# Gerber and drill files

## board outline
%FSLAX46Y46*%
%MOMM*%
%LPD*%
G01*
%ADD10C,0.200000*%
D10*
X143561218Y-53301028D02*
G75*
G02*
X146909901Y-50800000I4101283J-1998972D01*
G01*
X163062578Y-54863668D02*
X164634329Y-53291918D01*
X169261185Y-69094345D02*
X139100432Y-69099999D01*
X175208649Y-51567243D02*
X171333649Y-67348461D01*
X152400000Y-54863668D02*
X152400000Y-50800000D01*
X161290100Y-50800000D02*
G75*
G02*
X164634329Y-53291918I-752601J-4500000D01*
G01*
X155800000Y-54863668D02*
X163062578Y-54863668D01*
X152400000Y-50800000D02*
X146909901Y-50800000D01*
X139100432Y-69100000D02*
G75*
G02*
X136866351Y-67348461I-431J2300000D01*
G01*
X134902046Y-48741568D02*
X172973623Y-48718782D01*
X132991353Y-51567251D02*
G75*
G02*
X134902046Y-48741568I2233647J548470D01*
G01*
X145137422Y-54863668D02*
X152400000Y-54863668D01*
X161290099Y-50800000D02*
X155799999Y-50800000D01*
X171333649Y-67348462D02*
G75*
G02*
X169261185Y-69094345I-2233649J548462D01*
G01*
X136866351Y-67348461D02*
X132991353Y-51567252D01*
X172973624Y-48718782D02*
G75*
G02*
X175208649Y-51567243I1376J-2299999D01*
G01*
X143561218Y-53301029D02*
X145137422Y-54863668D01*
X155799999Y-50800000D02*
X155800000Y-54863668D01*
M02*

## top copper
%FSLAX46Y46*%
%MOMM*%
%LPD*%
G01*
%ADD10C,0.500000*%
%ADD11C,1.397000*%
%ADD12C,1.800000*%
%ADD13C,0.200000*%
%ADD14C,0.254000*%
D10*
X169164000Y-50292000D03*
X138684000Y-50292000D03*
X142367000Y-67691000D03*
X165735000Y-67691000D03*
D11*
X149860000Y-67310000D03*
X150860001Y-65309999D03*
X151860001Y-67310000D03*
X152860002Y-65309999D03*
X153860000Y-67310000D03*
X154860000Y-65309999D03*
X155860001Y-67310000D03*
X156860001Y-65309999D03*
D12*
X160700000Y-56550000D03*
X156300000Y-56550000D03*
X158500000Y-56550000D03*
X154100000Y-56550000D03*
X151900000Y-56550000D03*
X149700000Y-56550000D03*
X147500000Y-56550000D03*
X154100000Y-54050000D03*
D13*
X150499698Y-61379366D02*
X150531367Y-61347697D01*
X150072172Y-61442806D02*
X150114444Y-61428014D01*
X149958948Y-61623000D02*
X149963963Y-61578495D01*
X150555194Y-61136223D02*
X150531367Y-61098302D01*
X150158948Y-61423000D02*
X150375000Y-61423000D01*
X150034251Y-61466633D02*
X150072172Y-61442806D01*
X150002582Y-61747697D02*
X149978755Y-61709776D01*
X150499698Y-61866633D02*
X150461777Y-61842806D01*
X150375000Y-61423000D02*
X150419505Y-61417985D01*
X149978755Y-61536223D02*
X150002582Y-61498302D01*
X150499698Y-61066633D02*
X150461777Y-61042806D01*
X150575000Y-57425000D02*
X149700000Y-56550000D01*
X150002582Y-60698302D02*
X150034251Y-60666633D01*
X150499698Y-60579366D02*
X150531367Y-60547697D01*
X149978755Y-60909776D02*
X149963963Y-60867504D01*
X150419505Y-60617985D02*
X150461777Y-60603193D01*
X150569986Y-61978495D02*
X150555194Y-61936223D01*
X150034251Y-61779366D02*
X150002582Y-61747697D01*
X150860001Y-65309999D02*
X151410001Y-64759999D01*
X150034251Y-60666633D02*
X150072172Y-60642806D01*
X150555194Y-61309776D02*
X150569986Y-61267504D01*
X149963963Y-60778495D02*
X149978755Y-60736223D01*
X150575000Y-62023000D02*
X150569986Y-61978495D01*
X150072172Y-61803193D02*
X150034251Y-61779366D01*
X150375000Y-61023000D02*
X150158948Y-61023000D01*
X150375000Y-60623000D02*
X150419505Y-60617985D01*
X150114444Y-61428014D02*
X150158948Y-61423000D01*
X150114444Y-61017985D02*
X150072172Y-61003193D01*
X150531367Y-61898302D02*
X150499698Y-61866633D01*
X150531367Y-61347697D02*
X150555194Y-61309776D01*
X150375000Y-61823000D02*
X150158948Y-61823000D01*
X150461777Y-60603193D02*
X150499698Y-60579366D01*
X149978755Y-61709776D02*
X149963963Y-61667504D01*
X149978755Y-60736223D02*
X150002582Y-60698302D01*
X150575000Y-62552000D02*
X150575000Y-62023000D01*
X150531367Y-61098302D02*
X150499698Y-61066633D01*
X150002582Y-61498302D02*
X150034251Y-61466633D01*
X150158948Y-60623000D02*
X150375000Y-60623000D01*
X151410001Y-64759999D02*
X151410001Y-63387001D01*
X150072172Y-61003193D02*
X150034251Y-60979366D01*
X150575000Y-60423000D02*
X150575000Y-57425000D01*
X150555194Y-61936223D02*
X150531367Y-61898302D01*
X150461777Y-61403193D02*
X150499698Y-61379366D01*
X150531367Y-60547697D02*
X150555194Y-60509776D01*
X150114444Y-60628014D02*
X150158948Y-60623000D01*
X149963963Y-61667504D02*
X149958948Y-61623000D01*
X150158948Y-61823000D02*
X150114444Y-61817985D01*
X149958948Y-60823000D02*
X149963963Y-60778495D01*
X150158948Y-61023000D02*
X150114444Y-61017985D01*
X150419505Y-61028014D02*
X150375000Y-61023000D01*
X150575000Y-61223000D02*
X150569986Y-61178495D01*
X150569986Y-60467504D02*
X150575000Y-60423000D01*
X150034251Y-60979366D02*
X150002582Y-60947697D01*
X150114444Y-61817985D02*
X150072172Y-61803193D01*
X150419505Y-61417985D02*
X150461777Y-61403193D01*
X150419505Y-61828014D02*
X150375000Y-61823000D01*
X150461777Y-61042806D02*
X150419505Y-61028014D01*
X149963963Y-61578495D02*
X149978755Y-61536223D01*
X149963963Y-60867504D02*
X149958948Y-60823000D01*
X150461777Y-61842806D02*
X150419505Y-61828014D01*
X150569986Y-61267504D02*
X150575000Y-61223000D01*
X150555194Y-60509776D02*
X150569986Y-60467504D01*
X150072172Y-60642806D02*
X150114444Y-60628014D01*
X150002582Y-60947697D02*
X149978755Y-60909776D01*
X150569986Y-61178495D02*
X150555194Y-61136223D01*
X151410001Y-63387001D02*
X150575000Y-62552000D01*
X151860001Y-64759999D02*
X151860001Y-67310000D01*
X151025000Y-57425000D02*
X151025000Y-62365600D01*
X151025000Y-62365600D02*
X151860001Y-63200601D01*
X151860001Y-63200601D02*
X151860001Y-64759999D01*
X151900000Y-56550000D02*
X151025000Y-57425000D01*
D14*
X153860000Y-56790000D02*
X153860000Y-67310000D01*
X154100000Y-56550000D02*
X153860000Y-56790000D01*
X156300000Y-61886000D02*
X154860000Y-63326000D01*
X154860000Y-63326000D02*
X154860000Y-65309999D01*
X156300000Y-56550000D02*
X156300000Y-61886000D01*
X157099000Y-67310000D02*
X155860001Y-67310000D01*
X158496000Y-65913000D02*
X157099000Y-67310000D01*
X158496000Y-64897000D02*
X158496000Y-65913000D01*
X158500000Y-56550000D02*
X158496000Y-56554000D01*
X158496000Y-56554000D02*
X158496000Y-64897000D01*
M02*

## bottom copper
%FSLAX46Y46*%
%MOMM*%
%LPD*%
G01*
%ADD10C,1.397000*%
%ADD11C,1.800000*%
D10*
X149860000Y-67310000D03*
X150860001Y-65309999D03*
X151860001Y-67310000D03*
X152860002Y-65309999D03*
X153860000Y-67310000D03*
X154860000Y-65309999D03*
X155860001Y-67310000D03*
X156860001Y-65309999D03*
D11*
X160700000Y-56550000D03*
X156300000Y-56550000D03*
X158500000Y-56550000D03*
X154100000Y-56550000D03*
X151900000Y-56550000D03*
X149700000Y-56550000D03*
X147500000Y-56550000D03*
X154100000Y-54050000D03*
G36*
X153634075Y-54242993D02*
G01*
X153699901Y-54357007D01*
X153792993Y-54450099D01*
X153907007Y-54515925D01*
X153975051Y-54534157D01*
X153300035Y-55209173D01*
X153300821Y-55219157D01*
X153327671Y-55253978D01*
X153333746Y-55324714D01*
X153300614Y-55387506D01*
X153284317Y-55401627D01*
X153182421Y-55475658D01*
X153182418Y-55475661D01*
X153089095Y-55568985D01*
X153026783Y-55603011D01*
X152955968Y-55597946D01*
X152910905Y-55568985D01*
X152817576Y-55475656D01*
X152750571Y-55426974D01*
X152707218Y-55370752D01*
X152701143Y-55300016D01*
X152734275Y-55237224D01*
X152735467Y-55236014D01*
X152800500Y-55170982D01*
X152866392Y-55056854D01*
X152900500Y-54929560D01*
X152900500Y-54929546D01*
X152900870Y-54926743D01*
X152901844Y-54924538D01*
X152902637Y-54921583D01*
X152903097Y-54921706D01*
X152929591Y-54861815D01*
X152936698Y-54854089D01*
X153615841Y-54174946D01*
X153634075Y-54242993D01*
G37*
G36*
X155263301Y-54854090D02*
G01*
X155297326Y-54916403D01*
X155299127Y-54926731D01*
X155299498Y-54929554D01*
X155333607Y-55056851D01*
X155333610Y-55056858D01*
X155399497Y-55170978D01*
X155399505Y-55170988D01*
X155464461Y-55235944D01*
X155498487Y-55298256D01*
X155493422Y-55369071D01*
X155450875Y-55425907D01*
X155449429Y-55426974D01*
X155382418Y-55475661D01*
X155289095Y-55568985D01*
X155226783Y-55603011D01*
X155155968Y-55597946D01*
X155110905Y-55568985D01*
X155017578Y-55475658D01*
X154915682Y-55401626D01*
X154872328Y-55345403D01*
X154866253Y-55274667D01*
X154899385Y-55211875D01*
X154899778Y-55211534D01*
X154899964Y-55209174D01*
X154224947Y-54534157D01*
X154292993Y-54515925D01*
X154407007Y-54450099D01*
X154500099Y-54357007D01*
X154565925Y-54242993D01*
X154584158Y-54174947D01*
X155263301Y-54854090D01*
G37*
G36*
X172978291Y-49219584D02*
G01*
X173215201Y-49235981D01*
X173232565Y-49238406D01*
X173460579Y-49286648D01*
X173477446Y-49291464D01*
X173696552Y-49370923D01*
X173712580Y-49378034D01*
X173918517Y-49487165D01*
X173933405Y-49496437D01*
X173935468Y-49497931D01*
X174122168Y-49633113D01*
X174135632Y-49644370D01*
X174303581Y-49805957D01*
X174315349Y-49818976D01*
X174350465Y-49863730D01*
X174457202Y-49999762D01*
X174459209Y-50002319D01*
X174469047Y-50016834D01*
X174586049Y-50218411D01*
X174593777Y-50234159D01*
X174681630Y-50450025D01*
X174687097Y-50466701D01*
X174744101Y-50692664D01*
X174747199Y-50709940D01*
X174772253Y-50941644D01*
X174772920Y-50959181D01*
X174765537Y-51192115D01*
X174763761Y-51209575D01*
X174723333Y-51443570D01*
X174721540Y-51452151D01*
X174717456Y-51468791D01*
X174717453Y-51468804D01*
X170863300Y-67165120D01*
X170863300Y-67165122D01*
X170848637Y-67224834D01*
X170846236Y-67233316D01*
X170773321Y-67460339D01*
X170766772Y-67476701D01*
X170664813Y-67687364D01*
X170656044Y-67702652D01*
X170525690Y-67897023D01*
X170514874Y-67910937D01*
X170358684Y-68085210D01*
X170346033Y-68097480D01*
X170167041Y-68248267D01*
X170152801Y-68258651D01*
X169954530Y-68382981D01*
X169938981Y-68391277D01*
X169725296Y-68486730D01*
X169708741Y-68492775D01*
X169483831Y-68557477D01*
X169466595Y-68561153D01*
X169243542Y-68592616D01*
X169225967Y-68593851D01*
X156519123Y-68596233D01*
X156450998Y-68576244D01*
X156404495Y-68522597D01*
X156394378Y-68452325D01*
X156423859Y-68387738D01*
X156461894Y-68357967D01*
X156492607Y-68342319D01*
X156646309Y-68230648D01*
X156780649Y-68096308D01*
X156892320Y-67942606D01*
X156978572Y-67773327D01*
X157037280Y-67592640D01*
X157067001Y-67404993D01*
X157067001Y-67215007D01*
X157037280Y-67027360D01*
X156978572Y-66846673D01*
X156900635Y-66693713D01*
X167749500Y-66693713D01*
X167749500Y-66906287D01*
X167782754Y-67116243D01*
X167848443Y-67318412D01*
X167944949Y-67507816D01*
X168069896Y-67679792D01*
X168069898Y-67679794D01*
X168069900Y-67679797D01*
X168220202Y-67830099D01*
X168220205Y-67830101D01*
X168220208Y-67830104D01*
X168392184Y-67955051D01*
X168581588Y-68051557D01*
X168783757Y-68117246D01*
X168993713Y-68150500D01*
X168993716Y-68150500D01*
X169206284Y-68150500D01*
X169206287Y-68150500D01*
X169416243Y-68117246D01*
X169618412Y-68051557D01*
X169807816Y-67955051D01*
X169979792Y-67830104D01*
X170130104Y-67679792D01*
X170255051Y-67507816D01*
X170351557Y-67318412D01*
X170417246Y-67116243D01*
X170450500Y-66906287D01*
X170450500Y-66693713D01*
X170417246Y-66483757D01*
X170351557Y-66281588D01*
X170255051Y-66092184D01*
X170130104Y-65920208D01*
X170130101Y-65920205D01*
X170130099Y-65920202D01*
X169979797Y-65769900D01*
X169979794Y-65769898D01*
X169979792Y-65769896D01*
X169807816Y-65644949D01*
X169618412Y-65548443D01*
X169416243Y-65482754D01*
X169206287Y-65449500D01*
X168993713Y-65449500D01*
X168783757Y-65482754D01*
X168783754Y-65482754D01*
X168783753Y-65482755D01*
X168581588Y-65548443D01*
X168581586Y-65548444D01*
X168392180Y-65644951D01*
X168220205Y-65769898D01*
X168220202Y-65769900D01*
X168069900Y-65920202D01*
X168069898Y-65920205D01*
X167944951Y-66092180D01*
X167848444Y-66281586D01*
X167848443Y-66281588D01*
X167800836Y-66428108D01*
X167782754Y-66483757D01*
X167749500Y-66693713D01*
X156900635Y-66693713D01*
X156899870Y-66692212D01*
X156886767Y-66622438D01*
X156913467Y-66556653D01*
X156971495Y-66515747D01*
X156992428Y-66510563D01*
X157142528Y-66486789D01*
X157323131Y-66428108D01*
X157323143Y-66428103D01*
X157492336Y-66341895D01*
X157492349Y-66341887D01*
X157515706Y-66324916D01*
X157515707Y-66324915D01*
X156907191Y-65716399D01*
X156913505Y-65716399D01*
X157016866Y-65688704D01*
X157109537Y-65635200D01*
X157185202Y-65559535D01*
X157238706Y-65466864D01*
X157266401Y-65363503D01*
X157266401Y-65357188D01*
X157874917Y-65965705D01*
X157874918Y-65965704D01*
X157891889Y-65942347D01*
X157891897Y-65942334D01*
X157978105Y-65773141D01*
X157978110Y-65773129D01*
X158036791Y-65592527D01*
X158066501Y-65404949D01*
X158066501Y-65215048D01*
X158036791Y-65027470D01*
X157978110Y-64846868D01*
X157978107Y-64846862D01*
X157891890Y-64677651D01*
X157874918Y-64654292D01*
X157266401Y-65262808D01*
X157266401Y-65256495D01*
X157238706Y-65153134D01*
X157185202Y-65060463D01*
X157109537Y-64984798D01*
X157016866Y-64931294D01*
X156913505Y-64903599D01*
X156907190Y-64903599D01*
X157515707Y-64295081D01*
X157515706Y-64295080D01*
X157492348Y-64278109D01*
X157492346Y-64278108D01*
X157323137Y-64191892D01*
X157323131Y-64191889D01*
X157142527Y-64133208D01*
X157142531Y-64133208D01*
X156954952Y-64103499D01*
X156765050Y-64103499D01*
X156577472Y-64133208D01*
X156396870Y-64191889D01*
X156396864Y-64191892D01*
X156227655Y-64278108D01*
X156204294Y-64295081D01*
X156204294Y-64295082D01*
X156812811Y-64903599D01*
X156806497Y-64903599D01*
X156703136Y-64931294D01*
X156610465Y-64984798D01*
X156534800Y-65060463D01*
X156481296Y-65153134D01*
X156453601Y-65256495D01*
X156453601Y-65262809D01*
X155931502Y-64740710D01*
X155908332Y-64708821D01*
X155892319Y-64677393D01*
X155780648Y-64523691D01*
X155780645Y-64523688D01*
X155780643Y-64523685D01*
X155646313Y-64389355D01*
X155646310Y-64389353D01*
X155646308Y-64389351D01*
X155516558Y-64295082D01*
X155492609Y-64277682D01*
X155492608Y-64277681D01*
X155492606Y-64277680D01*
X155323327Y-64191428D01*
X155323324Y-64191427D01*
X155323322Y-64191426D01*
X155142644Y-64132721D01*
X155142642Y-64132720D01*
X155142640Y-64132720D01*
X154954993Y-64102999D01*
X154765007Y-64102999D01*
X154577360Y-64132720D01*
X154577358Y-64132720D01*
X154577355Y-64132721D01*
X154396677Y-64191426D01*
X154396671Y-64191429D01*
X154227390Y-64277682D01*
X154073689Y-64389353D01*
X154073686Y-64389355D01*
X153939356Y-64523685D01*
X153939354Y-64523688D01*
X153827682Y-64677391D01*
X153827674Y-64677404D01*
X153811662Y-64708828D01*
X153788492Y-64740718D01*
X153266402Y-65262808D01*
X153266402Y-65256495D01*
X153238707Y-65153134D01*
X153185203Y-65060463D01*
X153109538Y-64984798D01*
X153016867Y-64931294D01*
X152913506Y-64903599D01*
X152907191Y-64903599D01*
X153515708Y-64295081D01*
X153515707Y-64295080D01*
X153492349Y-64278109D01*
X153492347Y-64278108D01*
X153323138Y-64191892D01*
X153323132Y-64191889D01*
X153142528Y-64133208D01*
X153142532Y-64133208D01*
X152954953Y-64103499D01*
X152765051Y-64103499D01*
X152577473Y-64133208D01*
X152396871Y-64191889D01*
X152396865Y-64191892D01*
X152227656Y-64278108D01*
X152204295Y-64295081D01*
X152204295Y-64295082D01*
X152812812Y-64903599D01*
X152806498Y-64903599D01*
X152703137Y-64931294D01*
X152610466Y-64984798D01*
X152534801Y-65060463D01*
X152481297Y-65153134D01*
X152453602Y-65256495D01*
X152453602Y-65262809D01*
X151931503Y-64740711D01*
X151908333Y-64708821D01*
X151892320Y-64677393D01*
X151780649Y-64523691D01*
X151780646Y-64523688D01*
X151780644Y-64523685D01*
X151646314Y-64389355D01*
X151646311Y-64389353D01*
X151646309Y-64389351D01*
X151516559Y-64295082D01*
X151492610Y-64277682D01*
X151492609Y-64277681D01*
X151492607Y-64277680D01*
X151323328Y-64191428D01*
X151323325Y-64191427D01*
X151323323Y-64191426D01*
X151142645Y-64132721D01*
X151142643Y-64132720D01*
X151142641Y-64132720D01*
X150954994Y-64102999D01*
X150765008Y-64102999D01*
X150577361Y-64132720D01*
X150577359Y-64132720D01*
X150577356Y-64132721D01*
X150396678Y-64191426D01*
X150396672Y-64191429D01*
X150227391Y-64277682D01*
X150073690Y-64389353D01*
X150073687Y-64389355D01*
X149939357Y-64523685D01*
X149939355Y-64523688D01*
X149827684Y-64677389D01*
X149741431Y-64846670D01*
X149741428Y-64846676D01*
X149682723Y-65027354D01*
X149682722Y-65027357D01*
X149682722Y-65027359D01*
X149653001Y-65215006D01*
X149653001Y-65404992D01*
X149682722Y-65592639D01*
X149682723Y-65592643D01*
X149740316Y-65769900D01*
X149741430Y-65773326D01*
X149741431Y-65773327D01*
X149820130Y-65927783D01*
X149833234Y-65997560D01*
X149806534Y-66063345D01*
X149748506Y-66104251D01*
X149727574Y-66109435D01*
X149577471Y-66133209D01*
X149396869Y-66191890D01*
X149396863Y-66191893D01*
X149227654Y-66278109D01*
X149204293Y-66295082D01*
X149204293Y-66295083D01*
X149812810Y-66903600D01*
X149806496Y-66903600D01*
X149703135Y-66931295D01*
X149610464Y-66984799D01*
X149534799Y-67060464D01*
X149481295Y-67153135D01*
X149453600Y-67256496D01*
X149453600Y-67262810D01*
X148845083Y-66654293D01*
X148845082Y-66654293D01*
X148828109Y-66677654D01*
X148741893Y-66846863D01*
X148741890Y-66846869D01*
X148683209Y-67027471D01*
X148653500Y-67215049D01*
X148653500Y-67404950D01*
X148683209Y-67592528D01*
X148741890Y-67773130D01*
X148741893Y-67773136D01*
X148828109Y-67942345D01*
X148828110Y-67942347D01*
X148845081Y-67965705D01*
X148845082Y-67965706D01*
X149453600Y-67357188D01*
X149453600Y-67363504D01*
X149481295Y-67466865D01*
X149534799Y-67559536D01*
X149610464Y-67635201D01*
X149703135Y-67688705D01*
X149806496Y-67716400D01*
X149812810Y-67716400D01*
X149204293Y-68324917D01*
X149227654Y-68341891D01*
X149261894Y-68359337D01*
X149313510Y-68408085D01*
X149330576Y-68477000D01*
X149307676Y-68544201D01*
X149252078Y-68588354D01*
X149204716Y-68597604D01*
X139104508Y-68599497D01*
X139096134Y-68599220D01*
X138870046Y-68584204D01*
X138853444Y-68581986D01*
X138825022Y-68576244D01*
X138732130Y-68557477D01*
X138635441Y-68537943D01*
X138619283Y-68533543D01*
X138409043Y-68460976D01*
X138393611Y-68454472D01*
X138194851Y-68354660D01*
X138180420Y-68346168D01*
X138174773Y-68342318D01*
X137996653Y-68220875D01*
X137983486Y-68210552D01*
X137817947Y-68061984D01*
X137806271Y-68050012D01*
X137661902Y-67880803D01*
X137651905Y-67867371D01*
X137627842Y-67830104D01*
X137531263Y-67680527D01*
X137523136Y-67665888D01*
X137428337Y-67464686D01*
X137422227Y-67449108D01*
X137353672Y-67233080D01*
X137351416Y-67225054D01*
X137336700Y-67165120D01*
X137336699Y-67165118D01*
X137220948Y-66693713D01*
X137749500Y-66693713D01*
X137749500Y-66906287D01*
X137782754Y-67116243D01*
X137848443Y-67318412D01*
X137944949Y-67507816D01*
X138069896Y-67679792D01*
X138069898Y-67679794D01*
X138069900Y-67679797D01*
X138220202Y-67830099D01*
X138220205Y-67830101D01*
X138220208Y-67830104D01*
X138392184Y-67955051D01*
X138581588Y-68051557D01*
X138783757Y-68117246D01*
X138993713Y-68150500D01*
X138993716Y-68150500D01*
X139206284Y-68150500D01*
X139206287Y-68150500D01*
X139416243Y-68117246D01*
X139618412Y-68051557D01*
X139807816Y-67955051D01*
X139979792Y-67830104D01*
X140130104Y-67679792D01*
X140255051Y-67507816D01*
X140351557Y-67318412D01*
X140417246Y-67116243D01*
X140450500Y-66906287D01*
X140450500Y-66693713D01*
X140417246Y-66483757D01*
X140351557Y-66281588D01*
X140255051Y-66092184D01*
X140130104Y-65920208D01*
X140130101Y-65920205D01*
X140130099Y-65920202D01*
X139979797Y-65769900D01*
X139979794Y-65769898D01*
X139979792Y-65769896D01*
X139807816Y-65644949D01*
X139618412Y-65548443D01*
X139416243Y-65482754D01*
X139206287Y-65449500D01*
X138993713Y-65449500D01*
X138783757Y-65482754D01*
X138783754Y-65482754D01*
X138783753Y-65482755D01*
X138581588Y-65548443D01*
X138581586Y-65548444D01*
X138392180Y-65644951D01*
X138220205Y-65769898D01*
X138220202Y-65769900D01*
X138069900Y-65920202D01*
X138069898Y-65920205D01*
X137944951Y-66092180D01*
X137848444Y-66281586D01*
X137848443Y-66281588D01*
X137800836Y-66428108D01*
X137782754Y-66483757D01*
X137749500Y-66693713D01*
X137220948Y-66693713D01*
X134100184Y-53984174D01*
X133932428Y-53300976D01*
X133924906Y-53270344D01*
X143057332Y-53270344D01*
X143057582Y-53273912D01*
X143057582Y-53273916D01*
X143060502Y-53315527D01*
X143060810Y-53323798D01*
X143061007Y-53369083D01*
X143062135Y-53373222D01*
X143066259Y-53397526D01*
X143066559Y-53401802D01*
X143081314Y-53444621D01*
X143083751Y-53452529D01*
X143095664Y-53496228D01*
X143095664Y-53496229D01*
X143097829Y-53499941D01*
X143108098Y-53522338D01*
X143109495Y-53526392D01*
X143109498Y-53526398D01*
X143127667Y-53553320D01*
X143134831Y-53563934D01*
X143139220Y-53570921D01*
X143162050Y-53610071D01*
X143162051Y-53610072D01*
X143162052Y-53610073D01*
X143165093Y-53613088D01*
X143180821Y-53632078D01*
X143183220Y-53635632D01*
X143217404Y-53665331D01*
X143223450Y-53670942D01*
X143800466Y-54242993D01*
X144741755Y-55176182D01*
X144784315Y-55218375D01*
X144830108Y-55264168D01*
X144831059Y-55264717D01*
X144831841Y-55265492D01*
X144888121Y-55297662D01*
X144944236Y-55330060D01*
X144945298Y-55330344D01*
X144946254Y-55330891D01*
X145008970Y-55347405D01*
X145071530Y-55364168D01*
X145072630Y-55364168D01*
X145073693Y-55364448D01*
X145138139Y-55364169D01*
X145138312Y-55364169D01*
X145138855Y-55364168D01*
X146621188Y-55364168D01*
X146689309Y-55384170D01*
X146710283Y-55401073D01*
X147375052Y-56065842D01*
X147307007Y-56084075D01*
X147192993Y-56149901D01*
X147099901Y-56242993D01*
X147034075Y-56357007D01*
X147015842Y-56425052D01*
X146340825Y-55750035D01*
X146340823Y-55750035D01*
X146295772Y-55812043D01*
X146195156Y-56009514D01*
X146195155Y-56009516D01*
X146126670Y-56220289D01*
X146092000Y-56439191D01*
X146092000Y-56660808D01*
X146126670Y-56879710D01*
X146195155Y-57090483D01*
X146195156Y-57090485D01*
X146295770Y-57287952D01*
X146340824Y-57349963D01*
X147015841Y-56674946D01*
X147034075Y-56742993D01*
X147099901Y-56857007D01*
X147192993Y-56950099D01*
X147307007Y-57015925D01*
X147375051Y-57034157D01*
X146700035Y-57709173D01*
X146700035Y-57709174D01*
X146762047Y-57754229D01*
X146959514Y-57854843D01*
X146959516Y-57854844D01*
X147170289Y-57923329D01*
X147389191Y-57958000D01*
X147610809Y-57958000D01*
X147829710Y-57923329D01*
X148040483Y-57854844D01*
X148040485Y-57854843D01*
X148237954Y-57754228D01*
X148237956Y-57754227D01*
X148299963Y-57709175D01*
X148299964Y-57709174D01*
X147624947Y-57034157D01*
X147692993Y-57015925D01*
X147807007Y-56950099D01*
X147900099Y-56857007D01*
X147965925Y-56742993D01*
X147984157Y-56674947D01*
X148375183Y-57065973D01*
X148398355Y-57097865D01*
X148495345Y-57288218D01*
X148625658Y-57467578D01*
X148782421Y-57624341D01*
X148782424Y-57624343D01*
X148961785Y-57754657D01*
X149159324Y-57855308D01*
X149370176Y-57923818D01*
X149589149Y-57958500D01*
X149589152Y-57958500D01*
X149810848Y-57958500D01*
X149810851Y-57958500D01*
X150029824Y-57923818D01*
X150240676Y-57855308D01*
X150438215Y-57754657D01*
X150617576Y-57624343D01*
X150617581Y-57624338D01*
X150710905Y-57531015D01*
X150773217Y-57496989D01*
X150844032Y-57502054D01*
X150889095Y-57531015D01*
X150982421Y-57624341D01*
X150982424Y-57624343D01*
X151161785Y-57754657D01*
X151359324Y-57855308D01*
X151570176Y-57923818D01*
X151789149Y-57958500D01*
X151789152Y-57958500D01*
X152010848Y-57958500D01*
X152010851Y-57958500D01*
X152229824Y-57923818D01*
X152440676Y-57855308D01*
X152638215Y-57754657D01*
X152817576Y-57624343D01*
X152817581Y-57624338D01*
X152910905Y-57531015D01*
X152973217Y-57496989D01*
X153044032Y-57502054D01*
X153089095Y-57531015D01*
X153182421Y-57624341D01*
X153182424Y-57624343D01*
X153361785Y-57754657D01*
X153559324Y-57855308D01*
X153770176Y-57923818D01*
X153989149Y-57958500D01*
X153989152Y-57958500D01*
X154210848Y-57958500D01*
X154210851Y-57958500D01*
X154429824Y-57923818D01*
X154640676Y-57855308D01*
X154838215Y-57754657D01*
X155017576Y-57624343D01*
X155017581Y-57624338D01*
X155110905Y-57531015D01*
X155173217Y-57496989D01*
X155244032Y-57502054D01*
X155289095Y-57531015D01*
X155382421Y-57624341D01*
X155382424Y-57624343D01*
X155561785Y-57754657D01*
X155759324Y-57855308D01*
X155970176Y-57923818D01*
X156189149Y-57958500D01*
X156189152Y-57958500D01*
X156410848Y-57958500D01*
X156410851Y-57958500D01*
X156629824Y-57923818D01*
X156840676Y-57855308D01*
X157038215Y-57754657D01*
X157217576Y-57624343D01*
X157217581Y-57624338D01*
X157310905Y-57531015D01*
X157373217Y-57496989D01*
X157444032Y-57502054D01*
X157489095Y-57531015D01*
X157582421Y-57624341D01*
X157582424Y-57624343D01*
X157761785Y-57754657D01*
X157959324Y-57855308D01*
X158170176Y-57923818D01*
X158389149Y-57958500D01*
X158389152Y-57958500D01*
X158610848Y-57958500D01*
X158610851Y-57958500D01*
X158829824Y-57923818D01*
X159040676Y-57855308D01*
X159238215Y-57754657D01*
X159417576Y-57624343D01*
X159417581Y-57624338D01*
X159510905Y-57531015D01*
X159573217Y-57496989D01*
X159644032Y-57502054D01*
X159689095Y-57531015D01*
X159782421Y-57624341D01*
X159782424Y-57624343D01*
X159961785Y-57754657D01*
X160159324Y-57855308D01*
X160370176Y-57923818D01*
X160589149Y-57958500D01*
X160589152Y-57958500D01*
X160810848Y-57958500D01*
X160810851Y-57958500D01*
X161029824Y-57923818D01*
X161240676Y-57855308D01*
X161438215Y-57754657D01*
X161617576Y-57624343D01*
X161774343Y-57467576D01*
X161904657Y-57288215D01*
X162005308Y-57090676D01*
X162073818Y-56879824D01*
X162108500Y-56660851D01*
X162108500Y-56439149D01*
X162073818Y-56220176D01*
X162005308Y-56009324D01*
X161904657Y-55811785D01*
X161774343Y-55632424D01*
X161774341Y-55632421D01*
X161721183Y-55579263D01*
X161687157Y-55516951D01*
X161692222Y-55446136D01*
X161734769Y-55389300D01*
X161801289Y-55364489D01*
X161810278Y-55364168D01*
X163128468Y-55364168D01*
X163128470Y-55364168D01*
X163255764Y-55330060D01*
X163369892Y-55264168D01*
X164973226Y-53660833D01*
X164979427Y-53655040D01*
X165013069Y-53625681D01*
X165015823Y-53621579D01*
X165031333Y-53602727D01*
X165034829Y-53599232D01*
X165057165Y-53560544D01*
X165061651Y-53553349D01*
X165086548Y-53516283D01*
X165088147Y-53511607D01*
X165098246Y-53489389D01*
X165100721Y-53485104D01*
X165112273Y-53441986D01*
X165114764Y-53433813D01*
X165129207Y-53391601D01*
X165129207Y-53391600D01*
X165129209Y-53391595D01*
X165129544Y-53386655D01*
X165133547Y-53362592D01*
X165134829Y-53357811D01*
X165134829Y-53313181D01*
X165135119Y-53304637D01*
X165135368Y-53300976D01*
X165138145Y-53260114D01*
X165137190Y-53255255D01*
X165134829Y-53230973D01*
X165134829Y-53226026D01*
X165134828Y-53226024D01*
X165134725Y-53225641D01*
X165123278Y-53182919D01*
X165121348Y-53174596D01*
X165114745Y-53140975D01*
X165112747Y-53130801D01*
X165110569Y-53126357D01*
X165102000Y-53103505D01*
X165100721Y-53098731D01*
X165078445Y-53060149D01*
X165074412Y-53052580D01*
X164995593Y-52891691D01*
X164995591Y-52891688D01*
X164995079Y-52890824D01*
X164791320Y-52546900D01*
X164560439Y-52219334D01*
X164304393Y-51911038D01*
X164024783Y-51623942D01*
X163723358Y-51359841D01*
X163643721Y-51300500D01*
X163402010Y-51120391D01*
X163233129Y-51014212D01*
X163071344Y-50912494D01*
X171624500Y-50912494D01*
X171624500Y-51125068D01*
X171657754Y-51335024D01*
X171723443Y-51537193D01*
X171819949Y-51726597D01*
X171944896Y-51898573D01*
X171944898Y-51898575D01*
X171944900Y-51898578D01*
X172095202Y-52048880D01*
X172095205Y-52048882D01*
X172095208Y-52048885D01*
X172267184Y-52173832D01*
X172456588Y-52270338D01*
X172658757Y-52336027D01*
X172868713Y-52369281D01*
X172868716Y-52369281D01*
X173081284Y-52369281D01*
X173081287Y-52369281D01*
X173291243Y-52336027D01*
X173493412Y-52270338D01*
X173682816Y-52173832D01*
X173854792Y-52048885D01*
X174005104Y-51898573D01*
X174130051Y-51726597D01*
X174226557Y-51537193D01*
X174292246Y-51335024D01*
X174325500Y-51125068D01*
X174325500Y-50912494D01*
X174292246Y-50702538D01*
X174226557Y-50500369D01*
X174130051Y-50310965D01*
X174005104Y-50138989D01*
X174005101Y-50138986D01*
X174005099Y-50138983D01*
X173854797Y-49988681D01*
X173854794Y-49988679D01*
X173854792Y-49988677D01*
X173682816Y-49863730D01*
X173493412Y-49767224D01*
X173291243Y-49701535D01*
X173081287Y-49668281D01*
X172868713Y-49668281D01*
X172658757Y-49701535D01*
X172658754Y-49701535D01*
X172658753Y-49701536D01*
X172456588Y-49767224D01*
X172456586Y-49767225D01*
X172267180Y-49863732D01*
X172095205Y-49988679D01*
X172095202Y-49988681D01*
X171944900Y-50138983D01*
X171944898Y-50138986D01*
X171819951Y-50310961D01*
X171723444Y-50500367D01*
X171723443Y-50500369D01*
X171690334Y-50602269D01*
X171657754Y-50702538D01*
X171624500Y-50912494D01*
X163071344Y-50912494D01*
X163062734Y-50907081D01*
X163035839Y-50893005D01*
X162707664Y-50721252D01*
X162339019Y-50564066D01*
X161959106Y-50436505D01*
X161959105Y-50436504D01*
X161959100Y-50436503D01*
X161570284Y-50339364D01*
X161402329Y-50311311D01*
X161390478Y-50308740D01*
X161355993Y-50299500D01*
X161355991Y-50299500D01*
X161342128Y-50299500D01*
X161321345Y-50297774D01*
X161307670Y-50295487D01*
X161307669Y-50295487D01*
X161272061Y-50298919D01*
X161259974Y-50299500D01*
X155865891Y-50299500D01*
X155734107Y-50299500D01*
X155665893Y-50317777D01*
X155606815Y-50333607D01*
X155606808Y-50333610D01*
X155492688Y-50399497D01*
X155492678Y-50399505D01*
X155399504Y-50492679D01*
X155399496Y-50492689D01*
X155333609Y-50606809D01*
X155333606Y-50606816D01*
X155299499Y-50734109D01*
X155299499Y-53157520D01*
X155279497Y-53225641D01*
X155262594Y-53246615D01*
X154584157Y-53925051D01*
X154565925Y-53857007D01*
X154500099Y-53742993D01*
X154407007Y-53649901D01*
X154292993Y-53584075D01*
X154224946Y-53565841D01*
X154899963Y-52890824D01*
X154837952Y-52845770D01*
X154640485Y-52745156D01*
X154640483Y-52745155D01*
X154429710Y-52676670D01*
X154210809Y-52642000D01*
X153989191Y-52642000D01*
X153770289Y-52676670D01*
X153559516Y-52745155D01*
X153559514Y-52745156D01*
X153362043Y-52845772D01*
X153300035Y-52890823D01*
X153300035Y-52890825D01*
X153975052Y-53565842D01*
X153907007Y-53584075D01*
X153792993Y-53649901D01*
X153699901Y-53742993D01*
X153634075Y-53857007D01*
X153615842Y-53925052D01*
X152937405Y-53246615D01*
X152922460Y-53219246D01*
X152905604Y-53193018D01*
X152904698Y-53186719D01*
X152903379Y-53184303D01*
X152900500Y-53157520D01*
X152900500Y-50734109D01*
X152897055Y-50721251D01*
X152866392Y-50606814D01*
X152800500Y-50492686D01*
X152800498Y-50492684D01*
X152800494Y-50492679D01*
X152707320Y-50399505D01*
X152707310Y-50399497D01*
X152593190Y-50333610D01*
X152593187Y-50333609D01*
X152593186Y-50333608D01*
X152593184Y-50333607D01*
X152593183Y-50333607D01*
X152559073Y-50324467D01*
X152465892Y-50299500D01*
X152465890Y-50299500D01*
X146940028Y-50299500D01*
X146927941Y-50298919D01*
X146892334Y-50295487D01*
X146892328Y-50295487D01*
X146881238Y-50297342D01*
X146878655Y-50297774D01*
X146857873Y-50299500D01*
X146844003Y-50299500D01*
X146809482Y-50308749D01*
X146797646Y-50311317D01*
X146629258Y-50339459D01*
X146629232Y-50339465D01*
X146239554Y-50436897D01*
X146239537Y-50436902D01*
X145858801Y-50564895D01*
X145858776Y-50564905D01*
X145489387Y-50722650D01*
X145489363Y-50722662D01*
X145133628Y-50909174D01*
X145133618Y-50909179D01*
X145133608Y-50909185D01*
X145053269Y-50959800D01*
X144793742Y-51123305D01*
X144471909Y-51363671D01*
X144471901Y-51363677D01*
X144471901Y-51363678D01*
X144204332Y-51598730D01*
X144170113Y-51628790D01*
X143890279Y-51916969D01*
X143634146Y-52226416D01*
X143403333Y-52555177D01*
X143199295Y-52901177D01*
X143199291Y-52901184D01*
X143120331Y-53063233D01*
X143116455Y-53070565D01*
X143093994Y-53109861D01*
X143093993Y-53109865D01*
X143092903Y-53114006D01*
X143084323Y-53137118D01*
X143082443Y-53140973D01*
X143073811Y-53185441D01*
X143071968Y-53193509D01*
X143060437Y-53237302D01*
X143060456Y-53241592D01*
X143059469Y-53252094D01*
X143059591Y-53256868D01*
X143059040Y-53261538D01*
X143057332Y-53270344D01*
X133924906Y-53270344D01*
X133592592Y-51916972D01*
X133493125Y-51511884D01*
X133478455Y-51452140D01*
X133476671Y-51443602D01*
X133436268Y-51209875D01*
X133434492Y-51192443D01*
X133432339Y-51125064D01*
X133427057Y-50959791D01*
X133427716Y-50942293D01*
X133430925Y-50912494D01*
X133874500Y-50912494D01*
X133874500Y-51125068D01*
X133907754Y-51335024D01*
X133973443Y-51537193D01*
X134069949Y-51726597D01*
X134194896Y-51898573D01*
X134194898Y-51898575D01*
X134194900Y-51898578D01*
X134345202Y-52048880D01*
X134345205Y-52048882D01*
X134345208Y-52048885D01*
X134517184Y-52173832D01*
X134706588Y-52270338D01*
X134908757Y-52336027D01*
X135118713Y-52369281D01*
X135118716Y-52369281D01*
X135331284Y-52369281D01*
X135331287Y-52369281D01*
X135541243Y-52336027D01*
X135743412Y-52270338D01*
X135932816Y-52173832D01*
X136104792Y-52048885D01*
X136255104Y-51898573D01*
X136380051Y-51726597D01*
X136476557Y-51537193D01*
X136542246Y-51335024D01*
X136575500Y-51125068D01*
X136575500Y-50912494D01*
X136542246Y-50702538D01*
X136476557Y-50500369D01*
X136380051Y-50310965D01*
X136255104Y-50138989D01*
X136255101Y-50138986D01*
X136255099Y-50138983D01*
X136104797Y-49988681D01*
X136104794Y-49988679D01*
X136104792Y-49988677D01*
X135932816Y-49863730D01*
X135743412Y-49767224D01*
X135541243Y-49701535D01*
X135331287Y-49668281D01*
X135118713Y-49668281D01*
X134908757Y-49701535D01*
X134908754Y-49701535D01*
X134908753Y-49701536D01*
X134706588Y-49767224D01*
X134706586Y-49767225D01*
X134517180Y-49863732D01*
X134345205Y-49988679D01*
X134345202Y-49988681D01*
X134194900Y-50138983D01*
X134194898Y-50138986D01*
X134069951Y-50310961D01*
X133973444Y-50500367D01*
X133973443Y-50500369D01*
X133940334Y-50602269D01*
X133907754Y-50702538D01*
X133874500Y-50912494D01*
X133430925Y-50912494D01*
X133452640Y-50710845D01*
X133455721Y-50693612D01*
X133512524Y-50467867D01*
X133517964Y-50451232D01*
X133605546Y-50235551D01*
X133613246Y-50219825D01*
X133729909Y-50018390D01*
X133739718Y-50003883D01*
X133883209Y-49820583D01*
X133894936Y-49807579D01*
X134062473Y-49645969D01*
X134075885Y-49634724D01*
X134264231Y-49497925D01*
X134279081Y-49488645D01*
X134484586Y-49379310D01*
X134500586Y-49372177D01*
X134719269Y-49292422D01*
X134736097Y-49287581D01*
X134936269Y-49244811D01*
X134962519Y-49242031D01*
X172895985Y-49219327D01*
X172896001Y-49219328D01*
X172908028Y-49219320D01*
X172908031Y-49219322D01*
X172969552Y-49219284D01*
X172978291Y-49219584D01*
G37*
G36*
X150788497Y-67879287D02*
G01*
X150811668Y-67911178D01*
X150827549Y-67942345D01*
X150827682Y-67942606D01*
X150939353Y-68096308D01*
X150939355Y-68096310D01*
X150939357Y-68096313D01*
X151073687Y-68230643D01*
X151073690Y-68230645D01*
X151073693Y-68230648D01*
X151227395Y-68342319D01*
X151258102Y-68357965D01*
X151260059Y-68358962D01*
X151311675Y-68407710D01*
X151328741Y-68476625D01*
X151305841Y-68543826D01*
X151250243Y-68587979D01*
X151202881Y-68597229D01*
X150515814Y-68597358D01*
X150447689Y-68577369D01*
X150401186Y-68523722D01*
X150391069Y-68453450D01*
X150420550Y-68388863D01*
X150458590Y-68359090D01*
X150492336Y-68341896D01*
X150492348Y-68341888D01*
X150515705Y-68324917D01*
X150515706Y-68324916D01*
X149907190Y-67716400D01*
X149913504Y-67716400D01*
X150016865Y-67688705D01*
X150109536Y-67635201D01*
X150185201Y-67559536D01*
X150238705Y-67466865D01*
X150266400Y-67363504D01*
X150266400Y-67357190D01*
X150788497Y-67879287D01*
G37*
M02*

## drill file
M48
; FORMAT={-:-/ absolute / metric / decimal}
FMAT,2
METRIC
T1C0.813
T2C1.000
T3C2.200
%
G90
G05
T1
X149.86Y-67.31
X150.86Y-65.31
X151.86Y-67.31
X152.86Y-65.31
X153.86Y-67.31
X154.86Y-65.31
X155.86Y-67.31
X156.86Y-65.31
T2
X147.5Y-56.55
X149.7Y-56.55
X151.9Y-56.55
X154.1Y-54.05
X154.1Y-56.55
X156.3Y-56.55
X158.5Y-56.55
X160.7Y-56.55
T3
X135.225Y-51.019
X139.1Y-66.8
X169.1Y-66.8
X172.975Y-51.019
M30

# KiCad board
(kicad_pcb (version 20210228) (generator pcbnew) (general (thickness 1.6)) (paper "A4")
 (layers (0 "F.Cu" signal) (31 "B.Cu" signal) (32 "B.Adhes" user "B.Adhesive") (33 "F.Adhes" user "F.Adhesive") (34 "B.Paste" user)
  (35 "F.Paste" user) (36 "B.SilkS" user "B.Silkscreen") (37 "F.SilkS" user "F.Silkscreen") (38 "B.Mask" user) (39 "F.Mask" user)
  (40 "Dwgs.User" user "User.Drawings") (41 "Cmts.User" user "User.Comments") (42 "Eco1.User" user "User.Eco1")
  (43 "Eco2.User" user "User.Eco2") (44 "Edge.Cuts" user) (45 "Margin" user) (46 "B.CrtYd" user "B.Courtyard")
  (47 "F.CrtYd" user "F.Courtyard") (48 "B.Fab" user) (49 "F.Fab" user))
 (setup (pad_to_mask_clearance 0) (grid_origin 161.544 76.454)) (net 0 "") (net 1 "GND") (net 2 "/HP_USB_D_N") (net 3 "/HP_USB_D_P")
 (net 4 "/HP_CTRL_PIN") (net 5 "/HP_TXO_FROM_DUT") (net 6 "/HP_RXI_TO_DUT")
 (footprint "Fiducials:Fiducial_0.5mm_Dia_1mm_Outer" (layer "F.Cu") (at 169.164 50.292)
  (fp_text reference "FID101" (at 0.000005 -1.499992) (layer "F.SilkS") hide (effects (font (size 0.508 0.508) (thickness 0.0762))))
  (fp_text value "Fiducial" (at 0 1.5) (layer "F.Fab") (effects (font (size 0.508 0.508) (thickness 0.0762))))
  (pad "~" smd circle (at 0 0) (locked) (size 0.5 0.5) (layers "F.Cu" "F.Mask") (solder_mask_margin 0.25) (clearance 0.25)))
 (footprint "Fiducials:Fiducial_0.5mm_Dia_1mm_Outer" (layer "F.Cu") (at 138.684 50.292)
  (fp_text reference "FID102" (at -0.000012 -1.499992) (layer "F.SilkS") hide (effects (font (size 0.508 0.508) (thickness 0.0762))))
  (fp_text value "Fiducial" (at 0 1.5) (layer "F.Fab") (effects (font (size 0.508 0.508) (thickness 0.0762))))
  (pad "~" smd circle (at 0 0) (locked) (size 0.5 0.5) (layers "F.Cu" "F.Mask") (solder_mask_margin 0.25) (clearance 0.25)))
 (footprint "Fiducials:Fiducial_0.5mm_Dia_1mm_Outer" (layer "F.Cu") (at 142.367 67.691)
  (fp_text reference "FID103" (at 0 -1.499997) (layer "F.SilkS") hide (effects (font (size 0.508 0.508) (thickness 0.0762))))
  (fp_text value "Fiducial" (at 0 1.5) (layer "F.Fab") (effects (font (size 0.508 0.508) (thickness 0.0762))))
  (pad "~" smd circle (at 0 0) (locked) (size 0.5 0.5) (layers "F.Cu" "F.Mask") (solder_mask_margin 0.25) (clearance 0.25)))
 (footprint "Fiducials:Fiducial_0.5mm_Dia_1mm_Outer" (layer "F.Cu") (at 165.735 67.691)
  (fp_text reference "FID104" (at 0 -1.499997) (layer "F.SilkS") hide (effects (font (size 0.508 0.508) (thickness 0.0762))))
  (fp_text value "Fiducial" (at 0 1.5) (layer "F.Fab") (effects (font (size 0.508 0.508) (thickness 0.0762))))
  (pad "~" smd circle (at 0 0) (locked) (size 0.5 0.5) (layers "F.Cu" "F.Mask") (solder_mask_margin 0.25) (clearance 0.25)))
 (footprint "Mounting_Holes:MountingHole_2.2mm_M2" (layer "F.Cu") (at 135.225 51.018781)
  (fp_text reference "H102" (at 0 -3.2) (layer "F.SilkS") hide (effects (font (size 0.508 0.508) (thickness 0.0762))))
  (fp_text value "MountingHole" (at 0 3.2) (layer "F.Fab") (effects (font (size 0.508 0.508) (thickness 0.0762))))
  (pad "1" np_thru_hole circle (at 0 0) (locked) (size 2.2 2.2) (drill 2.2) (layers *.Cu *.Mask)))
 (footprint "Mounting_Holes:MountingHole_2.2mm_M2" (layer "F.Cu") (at 169.1 66.8)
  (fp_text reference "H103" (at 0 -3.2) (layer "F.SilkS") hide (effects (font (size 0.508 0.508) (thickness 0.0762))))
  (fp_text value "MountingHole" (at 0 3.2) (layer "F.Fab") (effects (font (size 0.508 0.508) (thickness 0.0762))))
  (pad "1" np_thru_hole circle (at 0 0) (locked) (size 2.2 2.2) (drill 2.2) (layers *.Cu *.Mask)))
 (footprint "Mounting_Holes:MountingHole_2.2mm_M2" (layer "F.Cu") (at 139.1 66.8)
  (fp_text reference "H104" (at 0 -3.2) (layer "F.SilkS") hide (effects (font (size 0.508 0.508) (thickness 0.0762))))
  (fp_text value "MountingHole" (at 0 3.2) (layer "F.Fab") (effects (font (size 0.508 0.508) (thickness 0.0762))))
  (pad "1" np_thru_hole circle (at 0 0) (locked) (size 2.2 2.2) (drill 2.2) (layers *.Cu *.Mask)))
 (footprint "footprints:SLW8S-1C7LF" (layer "F.Cu") (at 149.86 67.31)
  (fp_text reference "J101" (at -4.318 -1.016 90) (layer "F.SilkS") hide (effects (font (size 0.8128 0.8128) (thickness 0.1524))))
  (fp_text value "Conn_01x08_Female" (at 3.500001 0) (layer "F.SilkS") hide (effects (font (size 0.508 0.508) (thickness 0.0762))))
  (pad "1" thru_hole circle (at 0 0) (locked) (size 1.397 1.397) (drill 0.8128) (layers *.Cu *.Mask) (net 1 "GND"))
  (pad "2" thru_hole circle (at 1.000001 -2.000001) (locked) (size 1.397 1.397) (drill 0.8128) (layers *.Cu *.Mask) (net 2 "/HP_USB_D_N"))
  (pad "3" thru_hole circle (at 2.000001 0) (locked) (size 1.397 1.397) (drill 0.8128) (layers *.Cu *.Mask) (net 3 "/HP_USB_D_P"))
  (pad "4" thru_hole circle (at 3.000002 -2.000001) (locked) (size 1.397 1.397) (drill 0.8128) (layers *.Cu *.Mask) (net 1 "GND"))
  (pad "5" thru_hole circle (at 4 0) (locked) (size 1.397 1.397) (drill 0.8128) (layers *.Cu *.Mask) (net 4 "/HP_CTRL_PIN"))
  (pad "6" thru_hole circle (at 5 -2.000001) (locked) (size 1.397 1.397) (drill 0.8128) (layers *.Cu *.Mask) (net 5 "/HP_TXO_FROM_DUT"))
  (pad "7" thru_hole circle (at 6.000001 0) (locked) (size 1.397 1.397) (drill 0.8128) (layers *.Cu *.Mask) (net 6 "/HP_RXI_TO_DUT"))
  (pad "8" thru_hole circle (at 7.000001 -2.000001) (locked) (size 1.397 1.397) (drill 0.8128) (layers *.Cu *.Mask) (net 1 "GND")))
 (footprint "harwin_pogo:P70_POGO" (layer "F.Cu") (at 160.7 56.55)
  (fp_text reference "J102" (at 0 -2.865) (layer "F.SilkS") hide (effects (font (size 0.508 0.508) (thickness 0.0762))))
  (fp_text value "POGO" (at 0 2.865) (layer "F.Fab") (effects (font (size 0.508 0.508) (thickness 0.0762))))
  (pad "1" thru_hole circle (at 0 0) (locked) (size 1.8 1.8) (drill 1) (layers *.Cu *.Mask)))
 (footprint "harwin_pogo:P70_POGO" (layer "F.Cu") (at 156.3 56.55)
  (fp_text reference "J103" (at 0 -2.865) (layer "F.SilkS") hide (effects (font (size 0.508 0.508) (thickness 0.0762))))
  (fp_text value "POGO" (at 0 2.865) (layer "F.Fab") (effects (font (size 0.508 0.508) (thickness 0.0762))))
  (pad "1" thru_hole circle (at 0 0) (locked) (size 1.8 1.8) (drill 1) (layers *.Cu *.Mask) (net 5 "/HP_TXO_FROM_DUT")))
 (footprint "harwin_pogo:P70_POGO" (layer "F.Cu") (at 158.5 56.55)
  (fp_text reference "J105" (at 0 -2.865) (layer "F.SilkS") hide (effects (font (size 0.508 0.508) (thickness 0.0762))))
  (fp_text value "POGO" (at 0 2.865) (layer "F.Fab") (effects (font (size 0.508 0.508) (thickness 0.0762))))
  (pad "1" thru_hole circle (at 0 0) (locked) (size 1.8 1.8) (drill 1) (layers *.Cu *.Mask) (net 6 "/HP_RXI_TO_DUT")))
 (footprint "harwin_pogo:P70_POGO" (layer "F.Cu") (at 154.1 56.55)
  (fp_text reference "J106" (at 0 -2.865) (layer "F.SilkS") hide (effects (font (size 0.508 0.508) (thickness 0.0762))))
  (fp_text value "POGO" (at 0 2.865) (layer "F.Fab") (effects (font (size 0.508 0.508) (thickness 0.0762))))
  (pad "1" thru_hole circle (at 0 0) (locked) (size 1.8 1.8) (drill 1) (layers *.Cu *.Mask) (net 4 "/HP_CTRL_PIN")))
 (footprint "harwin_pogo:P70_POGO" (layer "F.Cu") (at 151.9 56.55)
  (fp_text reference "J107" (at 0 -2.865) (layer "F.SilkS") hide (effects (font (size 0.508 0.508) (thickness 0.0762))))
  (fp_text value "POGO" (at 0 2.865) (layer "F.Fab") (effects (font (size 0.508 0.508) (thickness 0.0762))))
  (pad "1" thru_hole circle (at 0 0) (locked) (size 1.8 1.8) (drill 1) (layers *.Cu *.Mask) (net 3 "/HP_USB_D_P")))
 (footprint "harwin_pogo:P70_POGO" (layer "F.Cu") (at 149.7 56.55)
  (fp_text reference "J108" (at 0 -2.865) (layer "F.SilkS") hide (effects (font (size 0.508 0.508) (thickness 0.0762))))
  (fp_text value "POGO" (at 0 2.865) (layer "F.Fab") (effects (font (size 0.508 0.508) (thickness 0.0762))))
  (pad "1" thru_hole circle (at 0 0) (locked) (size 1.8 1.8) (drill 1) (layers *.Cu *.Mask) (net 2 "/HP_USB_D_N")))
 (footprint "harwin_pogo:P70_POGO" (layer "F.Cu") (at 147.5 56.55)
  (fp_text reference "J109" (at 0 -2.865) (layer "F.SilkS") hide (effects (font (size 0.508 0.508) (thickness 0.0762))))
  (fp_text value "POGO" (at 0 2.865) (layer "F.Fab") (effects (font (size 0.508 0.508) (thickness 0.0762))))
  (pad "1" thru_hole circle (at 0 0) (locked) (size 1.8 1.8) (drill 1) (layers *.Cu *.Mask) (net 1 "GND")))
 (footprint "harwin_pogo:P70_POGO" (layer "F.Cu") (at 154.1 54.05)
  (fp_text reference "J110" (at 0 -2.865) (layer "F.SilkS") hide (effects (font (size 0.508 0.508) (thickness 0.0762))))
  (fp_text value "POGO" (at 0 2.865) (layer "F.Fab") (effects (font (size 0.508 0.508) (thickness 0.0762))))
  (pad "1" thru_hole circle (at 0 0) (locked) (size 1.8 1.8) (drill 1) (layers *.Cu *.Mask) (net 1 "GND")))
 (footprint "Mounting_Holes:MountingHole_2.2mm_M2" (layer "F.Cu") (at 172.975 51.018781)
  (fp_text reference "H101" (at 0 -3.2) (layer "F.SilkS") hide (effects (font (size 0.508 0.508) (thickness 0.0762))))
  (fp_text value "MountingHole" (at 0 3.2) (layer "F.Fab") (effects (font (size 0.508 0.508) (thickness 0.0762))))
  (pad "1" np_thru_hole circle (at 0 0) (locked) (size 2.2 2.2) (drill 2.2) (layers *.Cu *.Mask)))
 (gr_arc (start 147.662501 55.3) (end 146.909901 50.8) (angle -54.52079504) (layer "Edge.Cuts") (width 0.2))
 (gr_line (start 163.062578 54.863668) (end 164.634329 53.291918) (layer "Edge.Cuts") (width 0.2))
 (gr_line (start 169.261185 69.094345) (end 139.100432 69.099999) (layer "Edge.Cuts") (width 0.2))
 (gr_line (start 175.208649 51.567243) (end 171.333649 67.348461) (layer "Edge.Cuts") (width 0.2))
 (gr_line (start 152.4 54.863668) (end 152.4 50.8) (layer "Edge.Cuts") (width 0.2))
 (gr_arc (start 160.537499 55.3) (end 164.634329 53.291918) (angle -54.39344287) (layer "Edge.Cuts") (width 0.2))
 (gr_line (start 155.8 54.863668) (end 163.062578 54.863668) (layer "Edge.Cuts") (width 0.2))
 (gr_line (start 152.4 50.8) (end 146.909901 50.8) (layer "Edge.Cuts") (width 0.2))
 (gr_arc (start 139.100001 66.8) (end 136.866351 67.348461) (angle -76.21498565) (layer "Edge.Cuts") (width 0.2))
 (gr_line (start 134.902046 48.741568) (end 172.973623 48.718782) (layer "Edge.Cuts") (width 0.2))
 (gr_arc (start 135.225 51.018781) (end 134.902046 48.741568) (angle -95.72412582) (layer "Edge.Cuts") (width 0.2))
 (gr_line (start 145.137422 54.863668) (end 152.4 54.863668) (layer "Edge.Cuts") (width 0.2))
 (gr_line (start 161.290099 50.8) (end 155.799999 50.8) (layer "Edge.Cuts") (width 0.2))
 (gr_arc (start 169.1 66.8) (end 169.261185 69.094345) (angle -72.18561683) (layer "Edge.Cuts") (width 0.2))
 (gr_line (start 136.866351 67.348461) (end 132.991353 51.567252) (layer "Edge.Cuts") (width 0.2))
 (gr_arc (start 172.975 51.018781) (end 175.208649 51.567243) (angle -103.830049) (layer "Edge.Cuts") (width 0.2))
 (gr_line (start 143.561218 53.301029) (end 145.137422 54.863668) (layer "Edge.Cuts") (width 0.2))
 (gr_line (start 155.799999 50.8) (end 155.8 54.863668) (layer "Edge.Cuts") (width 0.2))
 (segment (start 150.499698 61.379366) (end 150.531367 61.347697) (width 0.2) (layer "F.Cu") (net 2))
 (segment (start 150.072172 61.442806) (end 150.114444 61.428014) (width 0.2) (layer "F.Cu") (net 2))
 (segment (start 149.958948 61.623) (end 149.963963 61.578495) (width 0.2) (layer "F.Cu") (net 2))
 (segment (start 150.555194 61.136223) (end 150.531367 61.098302) (width 0.2) (layer "F.Cu") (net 2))
 (segment (start 150.158948 61.423) (end 150.375 61.423) (width 0.2) (layer "F.Cu") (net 2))
 (segment (start 150.034251 61.466633) (end 150.072172 61.442806) (width 0.2) (layer "F.Cu") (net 2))
 (segment (start 150.002582 61.747697) (end 149.978755 61.709776) (width 0.2) (layer "F.Cu") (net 2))
 (segment (start 150.499698 61.866633) (end 150.461777 61.842806) (width 0.2) (layer "F.Cu") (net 2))
 (segment (start 150.375 61.423) (end 150.419505 61.417985) (width 0.2) (layer "F.Cu") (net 2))
 (segment (start 149.978755 61.536223) (end 150.002582 61.498302) (width 0.2) (layer "F.Cu") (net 2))
 (segment (start 150.499698 61.066633) (end 150.461777 61.042806) (width 0.2) (layer "F.Cu") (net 2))
 (segment (start 150.575 57.425) (end 149.7 56.55) (width 0.2) (layer "F.Cu") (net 2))
 (segment (start 150.002582 60.698302) (end 150.034251 60.666633) (width 0.2) (layer "F.Cu") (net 2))
 (segment (start 150.499698 60.579366) (end 150.531367 60.547697) (width 0.2) (layer "F.Cu") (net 2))
 (segment (start 149.978755 60.909776) (end 149.963963 60.867504) (width 0.2) (layer "F.Cu") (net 2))
 (segment (start 150.419505 60.617985) (end 150.461777 60.603193) (width 0.2) (layer "F.Cu") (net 2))
 (segment (start 150.569986 61.978495) (end 150.555194 61.936223) (width 0.2) (layer "F.Cu") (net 2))
 (segment (start 150.034251 61.779366) (end 150.002582 61.747697) (width 0.2) (layer "F.Cu") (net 2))
 (segment (start 150.860001 65.309999) (end 151.410001 64.759999) (width 0.2) (layer "F.Cu") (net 2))
 (segment (start 150.034251 60.666633) (end 150.072172 60.642806) (width 0.2) (layer "F.Cu") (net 2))
 (segment (start 150.555194 61.309776) (end 150.569986 61.267504) (width 0.2) (layer "F.Cu") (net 2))
 (segment (start 149.963963 60.778495) (end 149.978755 60.736223) (width 0.2) (layer "F.Cu") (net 2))
 (segment (start 150.575 62.023) (end 150.569986 61.978495) (width 0.2) (layer "F.Cu") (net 2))
 (segment (start 150.072172 61.803193) (end 150.034251 61.779366) (width 0.2) (layer "F.Cu") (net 2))
 (segment (start 150.375 61.023) (end 150.158948 61.023) (width 0.2) (layer "F.Cu") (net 2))
 (segment (start 150.375 60.623) (end 150.419505 60.617985) (width 0.2) (layer "F.Cu") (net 2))
 (segment (start 150.114444 61.428014) (end 150.158948 61.423) (width 0.2) (layer "F.Cu") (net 2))
 (segment (start 150.114444 61.017985) (end 150.072172 61.003193) (width 0.2) (layer "F.Cu") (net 2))
 (segment (start 150.531367 61.898302) (end 150.499698 61.866633) (width 0.2) (layer "F.Cu") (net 2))
 (segment (start 150.531367 61.347697) (end 150.555194 61.309776) (width 0.2) (layer "F.Cu") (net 2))
 (segment (start 150.375 61.823) (end 150.158948 61.823) (width 0.2) (layer "F.Cu") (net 2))
 (segment (start 150.461777 60.603193) (end 150.499698 60.579366) (width 0.2) (layer "F.Cu") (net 2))
 (segment (start 149.978755 61.709776) (end 149.963963 61.667504) (width 0.2) (layer "F.Cu") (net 2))
 (segment (start 149.978755 60.736223) (end 150.002582 60.698302) (width 0.2) (layer "F.Cu") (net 2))
 (segment (start 150.575 62.552) (end 150.575 62.023) (width 0.2) (layer "F.Cu") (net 2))
 (segment (start 150.531367 61.098302) (end 150.499698 61.066633) (width 0.2) (layer "F.Cu") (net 2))
 (segment (start 150.002582 61.498302) (end 150.034251 61.466633) (width 0.2) (layer "F.Cu") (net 2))
 (segment (start 150.158948 60.623) (end 150.375 60.623) (width 0.2) (layer "F.Cu") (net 2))
 (segment (start 151.410001 64.759999) (end 151.410001 63.387001) (width 0.2) (layer "F.Cu") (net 2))
 (segment (start 150.072172 61.003193) (end 150.034251 60.979366) (width 0.2) (layer "F.Cu") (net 2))
 (segment (start 150.575 60.423) (end 150.575 57.425) (width 0.2) (layer "F.Cu") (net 2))
 (segment (start 150.555194 61.936223) (end 150.531367 61.898302) (width 0.2) (layer "F.Cu") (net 2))
 (segment (start 150.461777 61.403193) (end 150.499698 61.379366) (width 0.2) (layer "F.Cu") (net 2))
 (segment (start 150.531367 60.547697) (end 150.555194 60.509776) (width 0.2) (layer "F.Cu") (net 2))
 (segment (start 150.114444 60.628014) (end 150.158948 60.623) (width 0.2) (layer "F.Cu") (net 2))
 (segment (start 149.963963 61.667504) (end 149.958948 61.623) (width 0.2) (layer "F.Cu") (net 2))
 (segment (start 150.158948 61.823) (end 150.114444 61.817985) (width 0.2) (layer "F.Cu") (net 2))
 (segment (start 149.958948 60.823) (end 149.963963 60.778495) (width 0.2) (layer "F.Cu") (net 2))
 (segment (start 150.158948 61.023) (end 150.114444 61.017985) (width 0.2) (layer "F.Cu") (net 2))
 (segment (start 150.419505 61.028014) (end 150.375 61.023) (width 0.2) (layer "F.Cu") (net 2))
 (segment (start 150.575 61.223) (end 150.569986 61.178495) (width 0.2) (layer "F.Cu") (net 2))
 (segment (start 150.569986 60.467504) (end 150.575 60.423) (width 0.2) (layer "F.Cu") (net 2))
 (segment (start 150.034251 60.979366) (end 150.002582 60.947697) (width 0.2) (layer "F.Cu") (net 2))
 (segment (start 150.114444 61.817985) (end 150.072172 61.803193) (width 0.2) (layer "F.Cu") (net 2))
 (segment (start 150.419505 61.417985) (end 150.461777 61.403193) (width 0.2) (layer "F.Cu") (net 2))
 (segment (start 150.419505 61.828014) (end 150.375 61.823) (width 0.2) (layer "F.Cu") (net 2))
 (segment (start 150.461777 61.042806) (end 150.419505 61.028014) (width 0.2) (layer "F.Cu") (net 2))
 (segment (start 149.963963 61.578495) (end 149.978755 61.536223) (width 0.2) (layer "F.Cu") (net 2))
 (segment (start 149.963963 60.867504) (end 149.958948 60.823) (width 0.2) (layer "F.Cu") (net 2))
 (segment (start 150.461777 61.842806) (end 150.419505 61.828014) (width 0.2) (layer "F.Cu") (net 2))
 (segment (start 150.569986 61.267504) (end 150.575 61.223) (width 0.2) (layer "F.Cu") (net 2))
 (segment (start 150.555194 60.509776) (end 150.569986 60.467504) (width 0.2) (layer "F.Cu") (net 2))
 (segment (start 150.072172 60.642806) (end 150.114444 60.628014) (width 0.2) (layer "F.Cu") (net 2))
 (segment (start 150.002582 60.947697) (end 149.978755 60.909776) (width 0.2) (layer "F.Cu") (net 2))
 (segment (start 150.569986 61.178495) (end 150.555194 61.136223) (width 0.2) (layer "F.Cu") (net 2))
 (segment (start 151.410001 63.387001) (end 150.575 62.552) (width 0.2) (layer "F.Cu") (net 2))
 (segment (start 151.860001 64.759999) (end 151.860001 67.31) (width 0.2) (layer "F.Cu") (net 3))
 (segment (start 151.025 57.425) (end 151.025 62.3656) (width 0.2) (layer "F.Cu") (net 3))
 (segment (start 151.025 62.3656) (end 151.860001 63.200601) (width 0.2) (layer "F.Cu") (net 3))
 (segment (start 151.860001 63.200601) (end 151.860001 64.759999) (width 0.2) (layer "F.Cu") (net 3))
 (segment (start 151.9 56.55) (end 151.025 57.425) (width 0.2) (layer "F.Cu") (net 3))
 (segment (start 153.86 56.79) (end 153.86 67.31) (width 0.254) (layer "F.Cu") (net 4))
 (segment (start 154.1 56.55) (end 153.86 56.79) (width 0.254) (layer "F.Cu") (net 4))
 (segment (start 156.3 61.886) (end 154.86 63.326) (width 0.254) (layer "F.Cu") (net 5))
 (segment (start 154.86 63.326) (end 154.86 65.309999) (width 0.254) (layer "F.Cu") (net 5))
 (segment (start 156.3 56.55) (end 156.3 61.886) (width 0.254) (layer "F.Cu") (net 5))
 (segment (start 157.099 67.31) (end 155.860001 67.31) (width 0.254) (layer "F.Cu") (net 6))
 (segment (start 158.496 65.913) (end 157.099 67.31) (width 0.254) (layer "F.Cu") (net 6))
 (segment (start 158.496 64.897) (end 158.496 65.913) (width 0.254) (layer "F.Cu") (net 6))
 (segment (start 158.5 56.55) (end 158.496 56.554) (width 0.254) (layer "F.Cu") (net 6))
 (segment (start 158.496 56.554) (end 158.496 64.897) (width 0.254) (layer "F.Cu") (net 6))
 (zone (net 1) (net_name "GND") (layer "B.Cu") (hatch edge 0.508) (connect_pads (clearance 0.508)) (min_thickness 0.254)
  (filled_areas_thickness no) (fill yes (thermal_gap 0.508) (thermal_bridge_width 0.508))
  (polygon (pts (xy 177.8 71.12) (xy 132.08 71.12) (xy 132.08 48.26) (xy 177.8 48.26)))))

